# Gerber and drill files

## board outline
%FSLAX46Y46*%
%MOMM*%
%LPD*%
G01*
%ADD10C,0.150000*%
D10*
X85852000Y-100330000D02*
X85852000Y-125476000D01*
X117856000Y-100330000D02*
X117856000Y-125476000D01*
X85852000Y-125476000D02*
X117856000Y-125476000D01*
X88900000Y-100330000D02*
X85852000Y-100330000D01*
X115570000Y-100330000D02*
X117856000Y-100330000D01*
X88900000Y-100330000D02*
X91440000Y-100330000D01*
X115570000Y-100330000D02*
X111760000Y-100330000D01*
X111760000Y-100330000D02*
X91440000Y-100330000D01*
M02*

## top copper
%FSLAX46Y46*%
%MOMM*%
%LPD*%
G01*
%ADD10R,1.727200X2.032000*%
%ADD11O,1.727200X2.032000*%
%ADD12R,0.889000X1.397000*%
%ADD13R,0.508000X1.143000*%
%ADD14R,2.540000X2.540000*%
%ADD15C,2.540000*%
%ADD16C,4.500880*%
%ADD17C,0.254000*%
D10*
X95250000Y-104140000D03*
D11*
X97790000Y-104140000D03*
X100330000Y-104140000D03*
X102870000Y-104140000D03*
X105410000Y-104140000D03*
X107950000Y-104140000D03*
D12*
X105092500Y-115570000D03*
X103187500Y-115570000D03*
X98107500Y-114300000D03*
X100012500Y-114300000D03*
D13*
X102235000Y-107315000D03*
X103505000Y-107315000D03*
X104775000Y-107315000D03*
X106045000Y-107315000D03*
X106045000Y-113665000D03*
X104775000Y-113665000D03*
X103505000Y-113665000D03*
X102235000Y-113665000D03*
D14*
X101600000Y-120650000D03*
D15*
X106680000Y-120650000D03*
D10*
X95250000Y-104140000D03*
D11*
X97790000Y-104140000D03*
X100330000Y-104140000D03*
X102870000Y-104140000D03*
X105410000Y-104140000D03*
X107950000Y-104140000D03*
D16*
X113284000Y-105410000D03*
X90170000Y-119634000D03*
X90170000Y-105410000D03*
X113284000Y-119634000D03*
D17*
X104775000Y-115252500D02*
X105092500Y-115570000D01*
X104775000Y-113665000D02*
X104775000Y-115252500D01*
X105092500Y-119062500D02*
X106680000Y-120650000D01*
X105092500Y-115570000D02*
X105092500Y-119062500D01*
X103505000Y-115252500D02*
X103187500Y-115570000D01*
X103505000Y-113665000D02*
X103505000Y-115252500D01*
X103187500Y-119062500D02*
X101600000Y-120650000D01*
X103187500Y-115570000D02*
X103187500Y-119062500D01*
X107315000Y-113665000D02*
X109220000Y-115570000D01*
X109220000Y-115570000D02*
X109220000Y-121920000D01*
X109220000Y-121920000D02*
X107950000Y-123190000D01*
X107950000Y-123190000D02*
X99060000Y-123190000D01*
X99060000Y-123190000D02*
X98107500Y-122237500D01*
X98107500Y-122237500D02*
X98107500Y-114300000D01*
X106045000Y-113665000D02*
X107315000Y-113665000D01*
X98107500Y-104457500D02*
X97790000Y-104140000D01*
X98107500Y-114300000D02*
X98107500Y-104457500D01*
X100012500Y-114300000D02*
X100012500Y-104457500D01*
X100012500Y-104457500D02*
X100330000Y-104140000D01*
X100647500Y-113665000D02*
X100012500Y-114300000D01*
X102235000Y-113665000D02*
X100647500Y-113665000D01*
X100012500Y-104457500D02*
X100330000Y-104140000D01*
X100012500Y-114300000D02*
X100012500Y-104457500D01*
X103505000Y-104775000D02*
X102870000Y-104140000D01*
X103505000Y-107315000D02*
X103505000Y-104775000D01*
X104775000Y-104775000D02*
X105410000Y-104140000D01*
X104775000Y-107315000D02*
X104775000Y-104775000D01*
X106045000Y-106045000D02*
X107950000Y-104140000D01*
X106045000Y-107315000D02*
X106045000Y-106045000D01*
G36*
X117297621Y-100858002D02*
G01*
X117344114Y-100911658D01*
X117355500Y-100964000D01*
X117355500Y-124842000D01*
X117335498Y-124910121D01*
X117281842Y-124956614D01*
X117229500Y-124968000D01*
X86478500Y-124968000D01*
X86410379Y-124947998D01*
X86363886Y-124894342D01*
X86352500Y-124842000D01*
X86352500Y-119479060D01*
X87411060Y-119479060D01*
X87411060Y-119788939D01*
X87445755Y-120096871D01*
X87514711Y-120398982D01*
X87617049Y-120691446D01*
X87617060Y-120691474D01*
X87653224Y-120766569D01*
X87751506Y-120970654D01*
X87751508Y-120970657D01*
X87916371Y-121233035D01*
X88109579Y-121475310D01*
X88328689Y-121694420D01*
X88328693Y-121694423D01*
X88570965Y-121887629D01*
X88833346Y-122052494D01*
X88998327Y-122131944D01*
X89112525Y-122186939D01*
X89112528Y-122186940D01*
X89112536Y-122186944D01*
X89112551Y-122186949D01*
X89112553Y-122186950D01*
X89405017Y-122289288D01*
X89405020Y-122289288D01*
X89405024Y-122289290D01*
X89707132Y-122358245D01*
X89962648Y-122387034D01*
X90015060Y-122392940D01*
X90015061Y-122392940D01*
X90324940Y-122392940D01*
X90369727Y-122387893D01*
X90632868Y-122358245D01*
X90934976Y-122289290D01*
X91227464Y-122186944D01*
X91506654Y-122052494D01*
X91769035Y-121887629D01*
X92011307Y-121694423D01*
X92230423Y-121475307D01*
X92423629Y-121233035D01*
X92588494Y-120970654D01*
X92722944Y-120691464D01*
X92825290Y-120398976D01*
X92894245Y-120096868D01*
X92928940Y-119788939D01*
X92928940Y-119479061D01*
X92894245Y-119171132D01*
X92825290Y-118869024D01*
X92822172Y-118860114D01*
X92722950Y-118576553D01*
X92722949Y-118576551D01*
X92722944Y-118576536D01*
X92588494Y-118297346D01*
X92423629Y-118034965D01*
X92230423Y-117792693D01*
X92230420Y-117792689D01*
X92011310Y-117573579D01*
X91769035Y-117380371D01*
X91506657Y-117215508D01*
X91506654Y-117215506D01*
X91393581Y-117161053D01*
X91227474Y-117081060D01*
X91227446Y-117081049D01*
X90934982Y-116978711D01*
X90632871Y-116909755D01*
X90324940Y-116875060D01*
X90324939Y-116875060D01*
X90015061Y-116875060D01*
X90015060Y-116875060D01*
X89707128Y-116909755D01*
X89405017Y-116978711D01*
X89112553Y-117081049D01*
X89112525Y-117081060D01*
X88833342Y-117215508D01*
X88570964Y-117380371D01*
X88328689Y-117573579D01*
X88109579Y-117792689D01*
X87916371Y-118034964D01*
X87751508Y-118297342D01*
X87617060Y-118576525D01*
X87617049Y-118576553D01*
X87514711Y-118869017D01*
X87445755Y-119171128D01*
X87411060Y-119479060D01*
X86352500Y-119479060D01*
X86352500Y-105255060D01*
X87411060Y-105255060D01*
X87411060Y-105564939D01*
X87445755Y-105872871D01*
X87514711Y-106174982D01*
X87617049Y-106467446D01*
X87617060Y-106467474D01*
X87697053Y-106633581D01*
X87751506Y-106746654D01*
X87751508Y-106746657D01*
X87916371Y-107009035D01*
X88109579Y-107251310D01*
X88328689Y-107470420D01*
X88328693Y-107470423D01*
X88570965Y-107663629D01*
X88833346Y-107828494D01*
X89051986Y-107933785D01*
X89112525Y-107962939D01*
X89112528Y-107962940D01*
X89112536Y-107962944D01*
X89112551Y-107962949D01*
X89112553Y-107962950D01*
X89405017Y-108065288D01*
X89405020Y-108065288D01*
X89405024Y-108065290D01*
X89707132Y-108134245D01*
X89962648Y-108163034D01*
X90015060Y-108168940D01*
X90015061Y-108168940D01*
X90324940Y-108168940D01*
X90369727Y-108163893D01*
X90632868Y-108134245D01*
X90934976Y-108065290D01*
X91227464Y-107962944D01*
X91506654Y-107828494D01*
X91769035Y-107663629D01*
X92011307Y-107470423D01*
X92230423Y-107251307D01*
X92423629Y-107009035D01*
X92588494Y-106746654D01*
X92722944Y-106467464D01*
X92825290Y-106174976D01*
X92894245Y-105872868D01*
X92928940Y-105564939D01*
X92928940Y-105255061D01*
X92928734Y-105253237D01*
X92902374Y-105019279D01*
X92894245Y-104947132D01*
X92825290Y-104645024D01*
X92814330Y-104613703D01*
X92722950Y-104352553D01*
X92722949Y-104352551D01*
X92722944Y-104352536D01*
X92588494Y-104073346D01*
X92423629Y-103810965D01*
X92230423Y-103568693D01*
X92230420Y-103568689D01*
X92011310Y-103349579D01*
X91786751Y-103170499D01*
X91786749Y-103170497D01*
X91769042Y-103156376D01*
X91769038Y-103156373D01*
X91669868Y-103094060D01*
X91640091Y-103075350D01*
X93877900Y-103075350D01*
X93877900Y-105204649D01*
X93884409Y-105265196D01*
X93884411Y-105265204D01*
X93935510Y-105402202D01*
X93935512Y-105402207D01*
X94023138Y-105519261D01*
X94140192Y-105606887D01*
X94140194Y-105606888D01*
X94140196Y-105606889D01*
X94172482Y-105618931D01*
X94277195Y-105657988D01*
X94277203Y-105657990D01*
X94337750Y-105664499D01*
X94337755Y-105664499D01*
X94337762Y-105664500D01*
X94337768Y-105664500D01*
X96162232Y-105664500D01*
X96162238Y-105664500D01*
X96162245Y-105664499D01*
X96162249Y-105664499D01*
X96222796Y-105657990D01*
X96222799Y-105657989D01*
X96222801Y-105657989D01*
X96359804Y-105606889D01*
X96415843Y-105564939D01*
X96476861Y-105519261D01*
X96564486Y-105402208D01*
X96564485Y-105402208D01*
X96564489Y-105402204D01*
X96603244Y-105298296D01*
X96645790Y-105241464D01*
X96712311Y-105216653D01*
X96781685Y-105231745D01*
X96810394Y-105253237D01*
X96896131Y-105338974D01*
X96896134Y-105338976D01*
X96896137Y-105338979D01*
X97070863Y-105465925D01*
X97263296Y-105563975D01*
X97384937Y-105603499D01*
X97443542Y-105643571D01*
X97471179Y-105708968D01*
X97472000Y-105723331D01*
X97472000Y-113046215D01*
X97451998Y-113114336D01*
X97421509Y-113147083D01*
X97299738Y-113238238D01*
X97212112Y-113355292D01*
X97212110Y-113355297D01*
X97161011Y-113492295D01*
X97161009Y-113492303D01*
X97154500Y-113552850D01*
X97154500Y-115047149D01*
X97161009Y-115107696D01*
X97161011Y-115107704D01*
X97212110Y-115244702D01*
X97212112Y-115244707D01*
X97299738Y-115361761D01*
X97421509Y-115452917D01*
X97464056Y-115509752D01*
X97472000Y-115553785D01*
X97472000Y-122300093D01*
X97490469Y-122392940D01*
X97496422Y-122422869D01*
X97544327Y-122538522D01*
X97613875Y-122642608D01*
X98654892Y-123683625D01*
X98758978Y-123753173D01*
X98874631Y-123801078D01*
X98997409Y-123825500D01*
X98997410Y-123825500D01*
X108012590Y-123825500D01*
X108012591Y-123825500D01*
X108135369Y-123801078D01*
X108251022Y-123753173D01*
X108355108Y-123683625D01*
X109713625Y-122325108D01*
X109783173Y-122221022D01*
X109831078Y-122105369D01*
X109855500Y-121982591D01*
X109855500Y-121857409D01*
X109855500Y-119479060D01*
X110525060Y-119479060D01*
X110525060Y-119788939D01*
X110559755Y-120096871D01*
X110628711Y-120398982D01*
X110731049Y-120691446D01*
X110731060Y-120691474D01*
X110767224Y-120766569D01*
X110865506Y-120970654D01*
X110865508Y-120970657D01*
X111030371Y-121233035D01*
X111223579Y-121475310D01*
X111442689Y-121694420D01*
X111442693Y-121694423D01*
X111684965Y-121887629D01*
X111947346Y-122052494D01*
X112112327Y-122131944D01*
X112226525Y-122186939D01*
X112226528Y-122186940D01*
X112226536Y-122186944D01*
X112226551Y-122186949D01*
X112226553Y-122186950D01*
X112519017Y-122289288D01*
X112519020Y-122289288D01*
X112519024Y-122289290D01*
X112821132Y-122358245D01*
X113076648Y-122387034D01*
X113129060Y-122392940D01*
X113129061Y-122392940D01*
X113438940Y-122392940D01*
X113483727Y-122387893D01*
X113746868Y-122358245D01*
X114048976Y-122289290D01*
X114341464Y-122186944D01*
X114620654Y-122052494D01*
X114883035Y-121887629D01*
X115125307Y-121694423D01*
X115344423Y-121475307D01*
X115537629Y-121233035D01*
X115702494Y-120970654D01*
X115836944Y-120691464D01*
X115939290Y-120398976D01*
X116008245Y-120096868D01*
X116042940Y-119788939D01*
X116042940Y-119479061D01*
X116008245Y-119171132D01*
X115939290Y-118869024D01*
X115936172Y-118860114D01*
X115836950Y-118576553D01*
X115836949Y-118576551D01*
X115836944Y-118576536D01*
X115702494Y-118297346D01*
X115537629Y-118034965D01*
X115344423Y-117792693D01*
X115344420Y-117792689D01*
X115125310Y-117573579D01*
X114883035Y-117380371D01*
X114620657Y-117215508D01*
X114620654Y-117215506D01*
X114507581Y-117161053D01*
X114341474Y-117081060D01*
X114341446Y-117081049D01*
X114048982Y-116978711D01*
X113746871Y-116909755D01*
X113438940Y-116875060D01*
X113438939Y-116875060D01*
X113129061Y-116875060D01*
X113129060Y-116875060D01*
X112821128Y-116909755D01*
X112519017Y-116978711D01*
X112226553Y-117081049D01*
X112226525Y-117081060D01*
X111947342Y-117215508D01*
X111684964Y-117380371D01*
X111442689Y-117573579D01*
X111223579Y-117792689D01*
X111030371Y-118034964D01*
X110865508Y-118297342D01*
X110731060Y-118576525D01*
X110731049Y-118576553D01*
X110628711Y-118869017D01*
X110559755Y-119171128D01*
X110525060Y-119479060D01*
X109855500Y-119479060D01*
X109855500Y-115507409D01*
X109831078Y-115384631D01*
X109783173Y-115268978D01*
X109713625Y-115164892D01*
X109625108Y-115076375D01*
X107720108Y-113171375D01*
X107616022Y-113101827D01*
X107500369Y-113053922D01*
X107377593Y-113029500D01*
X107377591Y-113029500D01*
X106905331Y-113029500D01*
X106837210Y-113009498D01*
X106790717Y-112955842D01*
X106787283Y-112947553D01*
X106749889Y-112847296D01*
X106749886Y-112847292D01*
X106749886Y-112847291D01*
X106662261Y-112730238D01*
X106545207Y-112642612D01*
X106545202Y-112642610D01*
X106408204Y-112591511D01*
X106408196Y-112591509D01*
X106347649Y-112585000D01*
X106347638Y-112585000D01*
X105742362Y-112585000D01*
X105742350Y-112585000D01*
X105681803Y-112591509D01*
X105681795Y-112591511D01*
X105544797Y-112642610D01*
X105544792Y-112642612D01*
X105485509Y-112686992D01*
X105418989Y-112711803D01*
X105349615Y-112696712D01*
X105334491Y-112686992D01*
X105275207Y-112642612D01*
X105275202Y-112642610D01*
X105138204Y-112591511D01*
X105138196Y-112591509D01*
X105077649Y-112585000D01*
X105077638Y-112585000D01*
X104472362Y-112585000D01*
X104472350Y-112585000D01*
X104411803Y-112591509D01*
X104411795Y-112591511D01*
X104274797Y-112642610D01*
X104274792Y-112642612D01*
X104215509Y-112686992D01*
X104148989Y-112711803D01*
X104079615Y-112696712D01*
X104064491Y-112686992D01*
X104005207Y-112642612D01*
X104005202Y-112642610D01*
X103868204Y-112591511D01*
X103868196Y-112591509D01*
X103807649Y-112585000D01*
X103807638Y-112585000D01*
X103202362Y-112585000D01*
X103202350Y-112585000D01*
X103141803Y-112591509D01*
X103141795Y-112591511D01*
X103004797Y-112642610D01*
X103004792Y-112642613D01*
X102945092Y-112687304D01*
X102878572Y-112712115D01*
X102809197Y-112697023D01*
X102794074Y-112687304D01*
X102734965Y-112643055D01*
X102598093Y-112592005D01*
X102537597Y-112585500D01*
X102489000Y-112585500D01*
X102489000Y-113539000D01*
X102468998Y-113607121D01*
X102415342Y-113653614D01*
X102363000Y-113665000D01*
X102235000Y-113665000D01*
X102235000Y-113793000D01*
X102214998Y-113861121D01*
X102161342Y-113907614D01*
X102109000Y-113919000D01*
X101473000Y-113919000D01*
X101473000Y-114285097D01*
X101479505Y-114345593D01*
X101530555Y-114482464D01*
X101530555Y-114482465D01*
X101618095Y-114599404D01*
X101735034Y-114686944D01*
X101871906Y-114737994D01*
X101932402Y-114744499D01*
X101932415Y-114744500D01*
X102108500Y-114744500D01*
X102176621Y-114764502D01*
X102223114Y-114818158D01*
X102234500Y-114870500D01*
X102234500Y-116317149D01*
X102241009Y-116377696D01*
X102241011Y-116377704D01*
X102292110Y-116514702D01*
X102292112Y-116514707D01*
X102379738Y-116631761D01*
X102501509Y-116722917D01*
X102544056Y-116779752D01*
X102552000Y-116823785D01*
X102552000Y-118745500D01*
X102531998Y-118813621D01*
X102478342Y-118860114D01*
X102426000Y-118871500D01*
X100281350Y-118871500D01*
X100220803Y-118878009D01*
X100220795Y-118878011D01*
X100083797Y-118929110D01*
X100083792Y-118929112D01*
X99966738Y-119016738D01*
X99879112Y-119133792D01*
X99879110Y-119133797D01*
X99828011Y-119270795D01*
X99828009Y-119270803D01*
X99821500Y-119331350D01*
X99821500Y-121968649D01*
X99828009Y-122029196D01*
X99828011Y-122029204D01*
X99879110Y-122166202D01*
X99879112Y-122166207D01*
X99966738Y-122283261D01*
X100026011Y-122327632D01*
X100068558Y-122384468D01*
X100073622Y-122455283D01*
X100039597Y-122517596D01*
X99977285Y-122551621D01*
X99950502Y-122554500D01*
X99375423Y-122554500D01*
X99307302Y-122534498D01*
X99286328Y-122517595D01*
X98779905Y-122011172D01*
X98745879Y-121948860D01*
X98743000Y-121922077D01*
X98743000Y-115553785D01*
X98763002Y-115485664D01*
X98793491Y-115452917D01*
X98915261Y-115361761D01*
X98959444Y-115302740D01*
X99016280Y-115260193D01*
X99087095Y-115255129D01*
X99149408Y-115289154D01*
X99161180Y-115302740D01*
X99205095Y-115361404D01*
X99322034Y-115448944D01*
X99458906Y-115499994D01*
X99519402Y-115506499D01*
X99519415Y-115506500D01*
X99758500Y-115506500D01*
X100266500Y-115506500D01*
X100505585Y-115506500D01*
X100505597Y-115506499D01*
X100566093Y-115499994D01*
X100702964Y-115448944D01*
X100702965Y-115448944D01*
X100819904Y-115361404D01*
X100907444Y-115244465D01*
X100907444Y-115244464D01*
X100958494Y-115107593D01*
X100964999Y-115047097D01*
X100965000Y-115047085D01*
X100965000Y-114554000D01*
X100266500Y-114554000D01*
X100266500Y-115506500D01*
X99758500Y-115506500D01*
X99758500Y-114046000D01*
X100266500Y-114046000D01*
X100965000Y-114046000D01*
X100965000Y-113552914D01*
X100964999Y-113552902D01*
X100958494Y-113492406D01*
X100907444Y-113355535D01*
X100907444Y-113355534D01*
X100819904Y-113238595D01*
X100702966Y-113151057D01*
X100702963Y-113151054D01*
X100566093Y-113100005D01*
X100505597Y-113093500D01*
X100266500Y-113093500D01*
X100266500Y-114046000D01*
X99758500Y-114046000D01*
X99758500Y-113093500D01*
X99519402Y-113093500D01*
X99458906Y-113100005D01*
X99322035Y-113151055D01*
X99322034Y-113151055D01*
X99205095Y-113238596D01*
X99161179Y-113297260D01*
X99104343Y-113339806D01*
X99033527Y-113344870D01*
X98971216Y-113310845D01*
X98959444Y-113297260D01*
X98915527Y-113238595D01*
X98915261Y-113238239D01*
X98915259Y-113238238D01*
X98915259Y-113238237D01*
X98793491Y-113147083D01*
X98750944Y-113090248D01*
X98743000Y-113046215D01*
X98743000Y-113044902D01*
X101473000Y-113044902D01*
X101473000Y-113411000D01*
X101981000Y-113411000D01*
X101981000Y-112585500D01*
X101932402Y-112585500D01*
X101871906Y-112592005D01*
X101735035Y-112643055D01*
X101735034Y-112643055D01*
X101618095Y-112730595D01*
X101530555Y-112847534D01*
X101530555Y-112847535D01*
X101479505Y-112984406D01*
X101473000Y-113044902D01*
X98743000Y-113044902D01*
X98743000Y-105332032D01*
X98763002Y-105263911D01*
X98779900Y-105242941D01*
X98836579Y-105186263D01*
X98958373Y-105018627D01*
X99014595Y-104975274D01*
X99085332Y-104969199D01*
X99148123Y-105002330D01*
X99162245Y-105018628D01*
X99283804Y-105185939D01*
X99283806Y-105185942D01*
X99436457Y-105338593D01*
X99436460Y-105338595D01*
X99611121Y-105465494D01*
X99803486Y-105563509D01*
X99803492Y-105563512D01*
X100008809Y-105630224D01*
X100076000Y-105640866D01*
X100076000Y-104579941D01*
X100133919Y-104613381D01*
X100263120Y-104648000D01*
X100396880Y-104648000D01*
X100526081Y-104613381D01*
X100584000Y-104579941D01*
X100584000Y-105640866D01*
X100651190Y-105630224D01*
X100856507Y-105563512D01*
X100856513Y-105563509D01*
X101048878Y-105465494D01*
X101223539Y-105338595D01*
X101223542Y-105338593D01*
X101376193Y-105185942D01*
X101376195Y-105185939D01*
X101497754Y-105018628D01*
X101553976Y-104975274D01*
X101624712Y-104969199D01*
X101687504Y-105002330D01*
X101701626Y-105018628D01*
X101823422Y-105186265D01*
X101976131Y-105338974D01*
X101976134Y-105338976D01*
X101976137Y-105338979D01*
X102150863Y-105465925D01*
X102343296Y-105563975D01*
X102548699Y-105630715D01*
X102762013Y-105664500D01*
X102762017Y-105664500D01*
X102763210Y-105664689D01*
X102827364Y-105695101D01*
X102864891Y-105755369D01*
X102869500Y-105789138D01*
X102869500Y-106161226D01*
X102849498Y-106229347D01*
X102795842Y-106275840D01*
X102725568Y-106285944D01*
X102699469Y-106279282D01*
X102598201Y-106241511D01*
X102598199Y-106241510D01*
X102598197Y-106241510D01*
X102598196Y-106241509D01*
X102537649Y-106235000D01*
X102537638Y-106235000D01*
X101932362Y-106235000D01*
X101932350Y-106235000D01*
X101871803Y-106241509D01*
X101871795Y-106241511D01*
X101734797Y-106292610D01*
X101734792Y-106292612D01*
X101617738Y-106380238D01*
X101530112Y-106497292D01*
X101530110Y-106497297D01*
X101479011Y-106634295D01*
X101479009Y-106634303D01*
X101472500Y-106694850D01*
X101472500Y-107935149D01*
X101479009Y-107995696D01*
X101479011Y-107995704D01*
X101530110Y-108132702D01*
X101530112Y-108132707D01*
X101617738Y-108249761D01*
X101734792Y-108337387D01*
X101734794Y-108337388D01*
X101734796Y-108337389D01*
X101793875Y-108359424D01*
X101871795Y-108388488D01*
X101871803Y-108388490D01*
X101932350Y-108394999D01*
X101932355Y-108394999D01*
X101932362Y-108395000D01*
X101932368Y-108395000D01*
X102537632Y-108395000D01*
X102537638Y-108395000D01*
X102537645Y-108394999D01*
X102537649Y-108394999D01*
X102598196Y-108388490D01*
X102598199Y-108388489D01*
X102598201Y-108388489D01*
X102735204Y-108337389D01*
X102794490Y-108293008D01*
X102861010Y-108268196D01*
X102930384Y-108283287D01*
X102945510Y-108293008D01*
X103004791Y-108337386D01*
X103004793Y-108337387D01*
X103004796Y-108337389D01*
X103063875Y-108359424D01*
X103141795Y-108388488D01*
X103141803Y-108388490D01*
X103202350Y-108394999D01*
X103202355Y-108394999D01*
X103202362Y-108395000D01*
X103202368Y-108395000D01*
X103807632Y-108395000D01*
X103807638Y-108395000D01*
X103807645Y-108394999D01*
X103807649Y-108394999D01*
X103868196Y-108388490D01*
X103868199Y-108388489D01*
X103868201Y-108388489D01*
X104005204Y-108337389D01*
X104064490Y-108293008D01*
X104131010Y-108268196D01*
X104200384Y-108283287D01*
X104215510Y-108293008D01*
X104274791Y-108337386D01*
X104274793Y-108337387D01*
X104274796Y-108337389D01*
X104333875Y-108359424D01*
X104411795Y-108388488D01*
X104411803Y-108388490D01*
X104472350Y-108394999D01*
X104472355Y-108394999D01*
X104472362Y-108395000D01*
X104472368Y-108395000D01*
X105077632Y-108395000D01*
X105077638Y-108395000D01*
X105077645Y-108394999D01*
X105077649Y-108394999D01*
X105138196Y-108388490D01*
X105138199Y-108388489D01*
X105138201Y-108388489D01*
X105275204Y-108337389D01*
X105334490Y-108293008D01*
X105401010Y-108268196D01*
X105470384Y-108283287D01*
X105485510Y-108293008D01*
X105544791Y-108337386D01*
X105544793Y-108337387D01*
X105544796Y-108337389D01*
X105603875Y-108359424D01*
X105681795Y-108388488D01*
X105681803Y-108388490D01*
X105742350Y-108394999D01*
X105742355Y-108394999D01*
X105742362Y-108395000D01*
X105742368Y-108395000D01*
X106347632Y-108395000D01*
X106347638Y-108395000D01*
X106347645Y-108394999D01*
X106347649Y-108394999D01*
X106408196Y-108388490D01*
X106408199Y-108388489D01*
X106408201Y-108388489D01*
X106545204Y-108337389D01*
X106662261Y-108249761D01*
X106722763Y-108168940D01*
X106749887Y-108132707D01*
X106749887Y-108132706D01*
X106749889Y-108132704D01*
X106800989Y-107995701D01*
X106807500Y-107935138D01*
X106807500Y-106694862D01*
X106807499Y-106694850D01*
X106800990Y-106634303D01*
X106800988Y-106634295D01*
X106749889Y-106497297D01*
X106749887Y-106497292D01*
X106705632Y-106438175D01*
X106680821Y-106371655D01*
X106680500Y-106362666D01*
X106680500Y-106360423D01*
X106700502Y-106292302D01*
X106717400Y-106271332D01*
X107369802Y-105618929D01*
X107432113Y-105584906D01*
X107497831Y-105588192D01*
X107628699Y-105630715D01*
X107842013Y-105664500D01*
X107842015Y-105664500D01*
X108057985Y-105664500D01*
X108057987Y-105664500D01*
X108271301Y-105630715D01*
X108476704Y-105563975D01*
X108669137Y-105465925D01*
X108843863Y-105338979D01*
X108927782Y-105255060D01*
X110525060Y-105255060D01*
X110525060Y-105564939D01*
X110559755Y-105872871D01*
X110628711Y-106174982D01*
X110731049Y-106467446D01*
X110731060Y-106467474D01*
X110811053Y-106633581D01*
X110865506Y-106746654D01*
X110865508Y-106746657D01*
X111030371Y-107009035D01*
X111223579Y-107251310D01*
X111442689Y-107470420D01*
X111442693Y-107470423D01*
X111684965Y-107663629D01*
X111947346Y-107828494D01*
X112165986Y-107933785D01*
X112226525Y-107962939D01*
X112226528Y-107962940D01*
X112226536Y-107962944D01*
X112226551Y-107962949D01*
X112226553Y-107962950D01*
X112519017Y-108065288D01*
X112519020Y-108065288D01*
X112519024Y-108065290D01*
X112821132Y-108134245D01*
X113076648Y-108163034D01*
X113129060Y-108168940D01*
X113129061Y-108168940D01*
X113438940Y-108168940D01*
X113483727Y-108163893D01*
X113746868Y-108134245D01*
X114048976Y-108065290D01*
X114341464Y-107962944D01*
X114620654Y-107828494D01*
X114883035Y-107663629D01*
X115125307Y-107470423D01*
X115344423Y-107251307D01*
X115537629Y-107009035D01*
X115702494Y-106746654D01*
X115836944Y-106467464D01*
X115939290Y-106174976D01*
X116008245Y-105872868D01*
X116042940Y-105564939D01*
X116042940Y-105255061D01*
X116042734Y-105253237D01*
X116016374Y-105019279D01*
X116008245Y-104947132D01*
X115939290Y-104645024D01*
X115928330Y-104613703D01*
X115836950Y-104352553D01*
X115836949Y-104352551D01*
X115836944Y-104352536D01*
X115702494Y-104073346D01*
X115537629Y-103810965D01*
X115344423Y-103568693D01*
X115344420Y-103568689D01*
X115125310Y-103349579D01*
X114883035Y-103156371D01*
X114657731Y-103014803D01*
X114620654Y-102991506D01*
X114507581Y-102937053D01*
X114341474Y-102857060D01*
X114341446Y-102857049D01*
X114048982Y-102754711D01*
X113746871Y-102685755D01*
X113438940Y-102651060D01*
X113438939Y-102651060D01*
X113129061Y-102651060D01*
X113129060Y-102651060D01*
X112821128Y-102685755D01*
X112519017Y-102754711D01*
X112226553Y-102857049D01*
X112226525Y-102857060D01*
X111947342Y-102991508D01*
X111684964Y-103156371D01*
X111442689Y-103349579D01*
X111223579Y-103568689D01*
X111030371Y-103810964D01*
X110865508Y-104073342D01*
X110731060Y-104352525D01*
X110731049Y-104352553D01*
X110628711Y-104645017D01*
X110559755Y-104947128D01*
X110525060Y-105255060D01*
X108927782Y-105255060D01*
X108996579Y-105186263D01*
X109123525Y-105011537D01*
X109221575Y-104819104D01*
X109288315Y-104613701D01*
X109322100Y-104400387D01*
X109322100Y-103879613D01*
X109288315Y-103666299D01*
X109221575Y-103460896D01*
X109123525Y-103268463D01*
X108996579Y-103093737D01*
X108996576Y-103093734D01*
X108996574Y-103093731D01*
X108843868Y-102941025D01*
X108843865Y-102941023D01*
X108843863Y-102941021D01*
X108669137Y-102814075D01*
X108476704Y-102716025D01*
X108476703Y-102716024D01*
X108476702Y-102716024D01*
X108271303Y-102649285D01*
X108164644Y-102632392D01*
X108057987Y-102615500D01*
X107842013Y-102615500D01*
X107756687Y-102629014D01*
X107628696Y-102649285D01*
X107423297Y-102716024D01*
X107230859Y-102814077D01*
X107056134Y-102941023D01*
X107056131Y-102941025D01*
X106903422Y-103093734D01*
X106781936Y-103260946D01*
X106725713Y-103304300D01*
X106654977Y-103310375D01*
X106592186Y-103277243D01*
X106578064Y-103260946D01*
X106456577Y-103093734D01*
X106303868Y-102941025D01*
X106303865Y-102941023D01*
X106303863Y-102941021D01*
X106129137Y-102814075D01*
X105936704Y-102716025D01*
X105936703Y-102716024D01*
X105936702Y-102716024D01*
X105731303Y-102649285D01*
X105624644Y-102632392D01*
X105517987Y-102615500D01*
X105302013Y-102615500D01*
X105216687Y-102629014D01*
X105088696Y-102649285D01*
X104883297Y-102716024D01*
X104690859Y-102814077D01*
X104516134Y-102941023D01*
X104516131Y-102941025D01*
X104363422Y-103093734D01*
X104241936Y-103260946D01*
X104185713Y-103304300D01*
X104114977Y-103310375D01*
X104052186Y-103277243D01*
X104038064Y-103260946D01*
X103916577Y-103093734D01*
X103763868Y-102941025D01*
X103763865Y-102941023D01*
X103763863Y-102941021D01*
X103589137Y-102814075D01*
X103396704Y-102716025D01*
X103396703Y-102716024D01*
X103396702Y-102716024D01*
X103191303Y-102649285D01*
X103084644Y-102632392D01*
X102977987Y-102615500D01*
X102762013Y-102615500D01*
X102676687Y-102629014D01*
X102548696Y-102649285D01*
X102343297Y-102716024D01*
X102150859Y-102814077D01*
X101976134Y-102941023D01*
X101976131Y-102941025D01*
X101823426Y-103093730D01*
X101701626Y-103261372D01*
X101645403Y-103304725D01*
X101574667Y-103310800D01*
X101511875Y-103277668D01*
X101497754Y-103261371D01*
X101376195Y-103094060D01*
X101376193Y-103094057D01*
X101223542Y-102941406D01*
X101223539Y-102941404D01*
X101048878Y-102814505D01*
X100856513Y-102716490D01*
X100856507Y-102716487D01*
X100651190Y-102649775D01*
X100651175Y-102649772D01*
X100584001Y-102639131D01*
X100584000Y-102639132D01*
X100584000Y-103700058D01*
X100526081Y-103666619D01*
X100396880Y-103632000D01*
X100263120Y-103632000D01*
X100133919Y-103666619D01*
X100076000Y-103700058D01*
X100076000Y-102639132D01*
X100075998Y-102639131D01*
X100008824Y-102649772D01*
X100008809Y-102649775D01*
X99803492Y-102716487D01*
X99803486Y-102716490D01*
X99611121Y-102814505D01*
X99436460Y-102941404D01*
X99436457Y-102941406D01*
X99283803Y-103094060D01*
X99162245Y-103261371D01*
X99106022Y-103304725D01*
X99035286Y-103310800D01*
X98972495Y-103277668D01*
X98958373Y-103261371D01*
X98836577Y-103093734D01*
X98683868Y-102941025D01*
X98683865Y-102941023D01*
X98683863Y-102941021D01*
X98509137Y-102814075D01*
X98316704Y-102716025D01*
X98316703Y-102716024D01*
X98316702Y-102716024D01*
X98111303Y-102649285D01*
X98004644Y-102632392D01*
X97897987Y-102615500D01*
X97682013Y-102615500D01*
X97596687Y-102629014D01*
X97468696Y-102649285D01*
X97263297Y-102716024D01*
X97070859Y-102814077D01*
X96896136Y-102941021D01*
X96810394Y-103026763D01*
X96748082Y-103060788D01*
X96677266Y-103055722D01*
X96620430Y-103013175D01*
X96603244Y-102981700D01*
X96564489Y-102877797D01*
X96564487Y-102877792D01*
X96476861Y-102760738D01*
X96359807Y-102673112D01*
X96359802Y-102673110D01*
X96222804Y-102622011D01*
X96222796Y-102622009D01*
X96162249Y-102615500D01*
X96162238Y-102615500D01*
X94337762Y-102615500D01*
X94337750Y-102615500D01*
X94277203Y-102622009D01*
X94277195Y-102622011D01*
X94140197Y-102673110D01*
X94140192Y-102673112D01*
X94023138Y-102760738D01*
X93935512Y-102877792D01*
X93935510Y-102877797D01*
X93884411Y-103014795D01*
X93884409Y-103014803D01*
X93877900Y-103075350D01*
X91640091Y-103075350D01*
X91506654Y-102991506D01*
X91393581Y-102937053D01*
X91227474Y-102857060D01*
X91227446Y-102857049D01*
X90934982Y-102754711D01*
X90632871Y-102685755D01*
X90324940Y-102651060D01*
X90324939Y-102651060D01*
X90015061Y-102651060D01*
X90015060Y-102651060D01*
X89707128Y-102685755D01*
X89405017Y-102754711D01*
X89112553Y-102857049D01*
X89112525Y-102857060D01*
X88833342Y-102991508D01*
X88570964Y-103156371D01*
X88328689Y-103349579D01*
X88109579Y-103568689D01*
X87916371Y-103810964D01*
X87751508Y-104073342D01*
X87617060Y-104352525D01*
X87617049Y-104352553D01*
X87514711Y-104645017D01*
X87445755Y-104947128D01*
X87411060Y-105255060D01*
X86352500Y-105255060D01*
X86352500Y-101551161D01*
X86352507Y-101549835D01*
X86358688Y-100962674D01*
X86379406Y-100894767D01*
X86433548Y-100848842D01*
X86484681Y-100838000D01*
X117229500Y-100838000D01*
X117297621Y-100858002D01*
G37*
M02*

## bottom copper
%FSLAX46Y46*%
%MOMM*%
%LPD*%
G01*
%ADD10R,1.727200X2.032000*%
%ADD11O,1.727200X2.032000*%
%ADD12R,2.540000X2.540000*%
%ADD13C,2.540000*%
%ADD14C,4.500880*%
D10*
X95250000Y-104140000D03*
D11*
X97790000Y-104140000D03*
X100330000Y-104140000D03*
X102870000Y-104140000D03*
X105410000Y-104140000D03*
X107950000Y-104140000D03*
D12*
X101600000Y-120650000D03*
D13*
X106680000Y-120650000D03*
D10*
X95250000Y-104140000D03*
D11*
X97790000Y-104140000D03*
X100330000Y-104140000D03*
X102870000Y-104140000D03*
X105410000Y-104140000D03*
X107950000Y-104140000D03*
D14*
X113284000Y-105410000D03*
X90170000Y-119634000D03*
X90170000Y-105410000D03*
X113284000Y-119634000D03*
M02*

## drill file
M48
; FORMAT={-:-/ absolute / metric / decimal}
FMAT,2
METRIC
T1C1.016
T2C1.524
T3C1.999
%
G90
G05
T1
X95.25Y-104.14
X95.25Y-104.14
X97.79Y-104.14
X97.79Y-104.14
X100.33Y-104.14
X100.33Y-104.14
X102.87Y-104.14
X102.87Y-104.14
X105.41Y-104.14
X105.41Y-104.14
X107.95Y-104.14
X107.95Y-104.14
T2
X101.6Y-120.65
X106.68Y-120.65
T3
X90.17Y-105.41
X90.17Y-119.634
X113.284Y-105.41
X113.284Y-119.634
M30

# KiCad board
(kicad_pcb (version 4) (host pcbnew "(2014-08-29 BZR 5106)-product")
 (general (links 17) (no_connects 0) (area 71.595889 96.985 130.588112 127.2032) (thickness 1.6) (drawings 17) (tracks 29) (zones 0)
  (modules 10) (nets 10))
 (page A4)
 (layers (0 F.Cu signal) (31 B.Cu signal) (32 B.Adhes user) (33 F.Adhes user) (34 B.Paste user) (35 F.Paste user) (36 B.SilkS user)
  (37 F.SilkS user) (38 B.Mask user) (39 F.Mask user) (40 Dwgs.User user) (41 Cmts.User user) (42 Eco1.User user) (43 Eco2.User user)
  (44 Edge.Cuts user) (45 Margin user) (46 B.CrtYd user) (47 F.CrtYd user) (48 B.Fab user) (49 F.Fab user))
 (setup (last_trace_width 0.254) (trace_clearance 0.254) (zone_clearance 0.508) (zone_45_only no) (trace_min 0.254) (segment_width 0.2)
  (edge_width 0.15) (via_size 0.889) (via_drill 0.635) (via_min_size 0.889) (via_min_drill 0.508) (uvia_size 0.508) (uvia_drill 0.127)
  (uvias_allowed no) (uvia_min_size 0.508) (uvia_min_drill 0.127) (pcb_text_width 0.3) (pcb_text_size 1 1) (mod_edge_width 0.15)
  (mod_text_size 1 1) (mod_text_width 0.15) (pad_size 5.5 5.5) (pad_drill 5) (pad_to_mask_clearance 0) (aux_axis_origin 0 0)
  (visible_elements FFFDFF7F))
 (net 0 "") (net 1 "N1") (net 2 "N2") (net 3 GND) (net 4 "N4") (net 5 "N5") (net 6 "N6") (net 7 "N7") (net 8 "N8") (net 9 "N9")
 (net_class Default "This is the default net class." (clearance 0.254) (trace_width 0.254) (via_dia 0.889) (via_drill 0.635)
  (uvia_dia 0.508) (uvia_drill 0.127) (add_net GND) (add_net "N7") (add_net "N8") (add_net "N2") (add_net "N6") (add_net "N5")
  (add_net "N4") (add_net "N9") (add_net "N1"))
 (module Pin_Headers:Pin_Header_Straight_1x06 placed (layer F.Cu) (at 101.6 104.14)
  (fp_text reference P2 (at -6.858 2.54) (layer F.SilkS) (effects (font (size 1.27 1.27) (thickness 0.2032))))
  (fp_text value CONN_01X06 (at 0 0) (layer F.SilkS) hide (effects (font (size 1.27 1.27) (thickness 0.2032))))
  (pad 1 thru_hole rect (at -6.35 0) (size 1.7272 2.032) (drill 1.016) (layers *.Cu *.Mask F.SilkS) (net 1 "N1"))
  (pad 2 thru_hole oval (at -3.81 0) (size 1.7272 2.032) (drill 1.016) (layers *.Cu *.Mask F.SilkS) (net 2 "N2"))
  (pad 3 thru_hole oval (at -1.27 0) (size 1.7272 2.032) (drill 1.016) (layers *.Cu *.Mask F.SilkS) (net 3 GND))
  (pad 4 thru_hole oval (at 1.27 0) (size 1.7272 2.032) (drill 1.016) (layers *.Cu *.Mask F.SilkS) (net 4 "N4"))
  (pad 5 thru_hole oval (at 3.81 0) (size 1.7272 2.032) (drill 1.016) (layers *.Cu *.Mask F.SilkS) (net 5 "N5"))
  (pad 6 thru_hole oval (at 6.35 0) (size 1.7272 2.032) (drill 1.016) (layers *.Cu *.Mask F.SilkS) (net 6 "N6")))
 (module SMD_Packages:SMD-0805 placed (layer F.Cu) (at 104.14 115.57 180)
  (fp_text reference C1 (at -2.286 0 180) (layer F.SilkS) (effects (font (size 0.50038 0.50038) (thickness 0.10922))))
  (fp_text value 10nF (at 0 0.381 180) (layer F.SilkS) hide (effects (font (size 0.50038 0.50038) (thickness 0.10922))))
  (pad 1 smd rect (at -0.9525 0 180) (size 0.889 1.397) (layers F.Cu F.Paste F.Mask) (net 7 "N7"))
  (pad 2 smd rect (at 0.9525 0 180) (size 0.889 1.397) (layers F.Cu F.Paste F.Mask) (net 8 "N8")))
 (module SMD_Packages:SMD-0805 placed (layer F.Cu) (at 99.06 114.3)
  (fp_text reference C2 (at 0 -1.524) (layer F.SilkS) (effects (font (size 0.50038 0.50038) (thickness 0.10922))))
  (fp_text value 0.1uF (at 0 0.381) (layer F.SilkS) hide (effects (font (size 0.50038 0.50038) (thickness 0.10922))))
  (pad 1 smd rect (at -0.9525 0) (size 0.889 1.397) (layers F.Cu F.Paste F.Mask) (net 2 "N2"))
  (pad 2 smd rect (at 0.9525 0) (size 0.889 1.397) (layers F.Cu F.Paste F.Mask) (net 3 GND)))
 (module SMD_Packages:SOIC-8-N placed (layer F.Cu) (at 104.14 110.49)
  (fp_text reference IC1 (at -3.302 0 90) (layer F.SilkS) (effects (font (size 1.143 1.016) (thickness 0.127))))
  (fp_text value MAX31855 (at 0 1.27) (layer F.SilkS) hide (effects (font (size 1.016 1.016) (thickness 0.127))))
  (pad 8 smd rect (at -1.905 -3.175) (size 0.508 1.143) (layers F.Cu F.Paste F.Mask) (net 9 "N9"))
  (pad 7 smd rect (at -0.635 -3.175) (size 0.508 1.143) (layers F.Cu F.Paste F.Mask) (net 4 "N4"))
  (pad 6 smd rect (at 0.635 -3.175) (size 0.508 1.143) (layers F.Cu F.Paste F.Mask) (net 5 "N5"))
  (pad 5 smd rect (at 1.905 -3.175) (size 0.508 1.143) (layers F.Cu F.Paste F.Mask) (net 6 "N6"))
  (pad 4 smd rect (at 1.905 3.175) (size 0.508 1.143) (layers F.Cu F.Paste F.Mask) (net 2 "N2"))
  (pad 3 smd rect (at 0.635 3.175) (size 0.508 1.143) (layers F.Cu F.Paste F.Mask) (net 7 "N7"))
  (pad 2 smd rect (at -0.635 3.175) (size 0.508 1.143) (layers F.Cu F.Paste F.Mask) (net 8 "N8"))
  (pad 1 smd rect (at -1.905 3.175) (size 0.508 1.143) (layers F.Cu F.Paste F.Mask) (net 3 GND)))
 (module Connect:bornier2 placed (layer F.Cu) (at 104.14 120.65)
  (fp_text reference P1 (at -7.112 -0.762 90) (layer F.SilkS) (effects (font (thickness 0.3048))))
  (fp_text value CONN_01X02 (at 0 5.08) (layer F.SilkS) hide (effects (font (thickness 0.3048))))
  (pad 1 thru_hole rect (at -2.54 0) (size 2.54 2.54) (drill 1.524) (layers *.Cu *.Mask F.SilkS) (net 8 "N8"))
  (pad 2 thru_hole circle (at 2.54 0) (size 2.54 2.54) (drill 1.524) (layers *.Cu *.Mask F.SilkS) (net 7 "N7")))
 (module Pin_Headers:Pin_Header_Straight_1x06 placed (layer F.Cu) (at 101.6 104.14)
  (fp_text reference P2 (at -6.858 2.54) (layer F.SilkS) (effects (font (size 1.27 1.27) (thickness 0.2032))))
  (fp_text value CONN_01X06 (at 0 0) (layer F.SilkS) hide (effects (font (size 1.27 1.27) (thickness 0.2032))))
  (pad 1 thru_hole rect (at -6.35 0) (size 1.7272 2.032) (drill 1.016) (layers *.Cu *.Mask F.SilkS) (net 1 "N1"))
  (pad 2 thru_hole oval (at -3.81 0) (size 1.7272 2.032) (drill 1.016) (layers *.Cu *.Mask F.SilkS) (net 2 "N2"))
  (pad 3 thru_hole oval (at -1.27 0) (size 1.7272 2.032) (drill 1.016) (layers *.Cu *.Mask F.SilkS) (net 3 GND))
  (pad 4 thru_hole oval (at 1.27 0) (size 1.7272 2.032) (drill 1.016) (layers *.Cu *.Mask F.SilkS) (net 4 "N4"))
  (pad 5 thru_hole oval (at 3.81 0) (size 1.7272 2.032) (drill 1.016) (layers *.Cu *.Mask F.SilkS) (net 5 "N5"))
  (pad 6 thru_hole oval (at 6.35 0) (size 1.7272 2.032) (drill 1.016) (layers *.Cu *.Mask F.SilkS) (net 6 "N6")))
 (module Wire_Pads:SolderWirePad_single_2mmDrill (layer F.Cu) (at 113.284 105.41)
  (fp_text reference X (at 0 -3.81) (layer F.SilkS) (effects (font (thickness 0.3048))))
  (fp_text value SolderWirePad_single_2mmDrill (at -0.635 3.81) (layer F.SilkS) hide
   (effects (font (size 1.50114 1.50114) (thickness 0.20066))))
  (pad 1 thru_hole circle (at 0 0) (size 4.50088 4.50088) (drill 1.99898) (layers *.Cu *.Mask F.SilkS)))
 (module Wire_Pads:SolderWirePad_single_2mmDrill (layer F.Cu) (at 90.17 119.634)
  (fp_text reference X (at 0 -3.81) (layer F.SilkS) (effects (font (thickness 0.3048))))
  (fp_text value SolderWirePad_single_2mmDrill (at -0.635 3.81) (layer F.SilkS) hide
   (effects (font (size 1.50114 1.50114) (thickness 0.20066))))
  (pad 1 thru_hole circle (at 0 0) (size 4.50088 4.50088) (drill 1.99898) (layers *.Cu *.Mask F.SilkS)))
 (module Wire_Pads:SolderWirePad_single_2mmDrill (layer F.Cu) (at 90.17 105.41)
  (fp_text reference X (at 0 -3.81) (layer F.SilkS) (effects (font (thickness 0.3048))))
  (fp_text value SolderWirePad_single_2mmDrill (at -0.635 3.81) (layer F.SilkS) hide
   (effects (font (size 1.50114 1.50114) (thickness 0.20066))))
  (pad 1 thru_hole circle (at 0 0) (size 4.50088 4.50088) (drill 1.99898) (layers *.Cu *.Mask F.SilkS)))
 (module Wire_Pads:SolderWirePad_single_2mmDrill (layer F.Cu) (at 113.284 119.634)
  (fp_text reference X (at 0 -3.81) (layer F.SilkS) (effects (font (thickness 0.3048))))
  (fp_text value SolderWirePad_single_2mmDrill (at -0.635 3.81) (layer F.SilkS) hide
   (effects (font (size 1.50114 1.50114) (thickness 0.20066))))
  (pad 1 thru_hole circle (at 0 0) (size 4.50088 4.50088) (drill 1.99898) (layers *.Cu *.Mask F.SilkS)))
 (gr_line (start 85.852 100.33) (end 85.852 125.476) (angle 90) (layer Edge.Cuts) (width 0.15))
 (gr_line (start 117.856 100.33) (end 117.856 125.476) (angle 90) (layer Edge.Cuts) (width 0.15))
 (gr_line (start 85.852 125.476) (end 117.856 125.476) (angle 90) (layer Edge.Cuts) (width 0.15))
 (gr_line (start 88.9 100.33) (end 85.852 100.33) (angle 90) (layer Edge.Cuts) (width 0.15))
 (gr_line (start 115.57 100.33) (end 117.856 100.33) (angle 90) (layer Edge.Cuts) (width 0.15))
 (gr_line (start 88.9 100.33) (end 91.44 100.33) (angle 90) (layer Edge.Cuts) (width 0.15))
 (gr_line (start 115.57 100.33) (end 111.76 100.33) (angle 90) (layer Edge.Cuts) (width 0.15))
 (gr_line (start 111.76 100.33) (end 91.44 100.33) (angle 90) (layer Edge.Cuts) (width 0.15))
 (segment (start 104.775 115.2525) (end 105.0925 115.57) (width 0.254) (layer F.Cu) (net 7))
 (segment (start 104.775 113.665) (end 104.775 115.2525) (width 0.254) (layer F.Cu) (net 7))
 (segment (start 105.0925 119.0625) (end 106.68 120.65) (width 0.254) (layer F.Cu) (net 7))
 (segment (start 105.0925 115.57) (end 105.0925 119.0625) (width 0.254) (layer F.Cu) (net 7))
 (segment (start 103.505 115.2525) (end 103.1875 115.57) (width 0.254) (layer F.Cu) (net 8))
 (segment (start 103.505 113.665) (end 103.505 115.2525) (width 0.254) (layer F.Cu) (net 8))
 (segment (start 103.1875 119.0625) (end 101.6 120.65) (width 0.254) (layer F.Cu) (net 8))
 (segment (start 103.1875 115.57) (end 103.1875 119.0625) (width 0.254) (layer F.Cu) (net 8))
 (segment (start 107.315 113.665) (end 109.22 115.57) (width 0.254) (layer F.Cu) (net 2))
 (segment (start 109.22 115.57) (end 109.22 121.92) (width 0.254) (layer F.Cu) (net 2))
 (segment (start 109.22 121.92) (end 107.95 123.19) (width 0.254) (layer F.Cu) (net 2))
 (segment (start 107.95 123.19) (end 99.06 123.19) (width 0.254) (layer F.Cu) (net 2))
 (segment (start 99.06 123.19) (end 98.1075 122.2375) (width 0.254) (layer F.Cu) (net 2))
 (segment (start 98.1075 122.2375) (end 98.1075 114.3) (width 0.254) (layer F.Cu) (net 2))
 (segment (start 106.045 113.665) (end 107.315 113.665) (width 0.254) (layer F.Cu) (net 2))
 (segment (start 98.1075 104.4575) (end 97.79 104.14) (width 0.254) (layer F.Cu) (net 2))
 (segment (start 98.1075 114.3) (end 98.1075 104.4575) (width 0.254) (layer F.Cu) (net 2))
 (segment (start 100.0125 114.3) (end 100.0125 104.4575) (width 0.254) (layer F.Cu) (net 3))
 (segment (start 100.0125 104.4575) (end 100.33 104.14) (width 0.254) (layer F.Cu) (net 3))
 (segment (start 100.6475 113.665) (end 100.0125 114.3) (width 0.254) (layer F.Cu) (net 3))
 (segment (start 102.235 113.665) (end 100.6475 113.665) (width 0.254) (layer F.Cu) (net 3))
 (segment (start 100.0125 104.4575) (end 100.33 104.14) (width 0.254) (layer F.Cu) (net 3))
 (segment (start 100.0125 114.3) (end 100.0125 104.4575) (width 0.254) (layer F.Cu) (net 3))
 (segment (start 103.505 104.775) (end 102.87 104.14) (width 0.254) (layer F.Cu) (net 4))
 (segment (start 103.505 107.315) (end 103.505 104.775) (width 0.254) (layer F.Cu) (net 4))
 (segment (start 104.775 104.775) (end 105.41 104.14) (width 0.254) (layer F.Cu) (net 5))
 (segment (start 104.775 107.315) (end 104.775 104.775) (width 0.254) (layer F.Cu) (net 5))
 (segment (start 106.045 106.045) (end 107.95 104.14) (width 0.254) (layer F.Cu) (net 6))
 (segment (start 106.045 107.315) (end 106.045 106.045) (width 0.254) (layer F.Cu) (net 6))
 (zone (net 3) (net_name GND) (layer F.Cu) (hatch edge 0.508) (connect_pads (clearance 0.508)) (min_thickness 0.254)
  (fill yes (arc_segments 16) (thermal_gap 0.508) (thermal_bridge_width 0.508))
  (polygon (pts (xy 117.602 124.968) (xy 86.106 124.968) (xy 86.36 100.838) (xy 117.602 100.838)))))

